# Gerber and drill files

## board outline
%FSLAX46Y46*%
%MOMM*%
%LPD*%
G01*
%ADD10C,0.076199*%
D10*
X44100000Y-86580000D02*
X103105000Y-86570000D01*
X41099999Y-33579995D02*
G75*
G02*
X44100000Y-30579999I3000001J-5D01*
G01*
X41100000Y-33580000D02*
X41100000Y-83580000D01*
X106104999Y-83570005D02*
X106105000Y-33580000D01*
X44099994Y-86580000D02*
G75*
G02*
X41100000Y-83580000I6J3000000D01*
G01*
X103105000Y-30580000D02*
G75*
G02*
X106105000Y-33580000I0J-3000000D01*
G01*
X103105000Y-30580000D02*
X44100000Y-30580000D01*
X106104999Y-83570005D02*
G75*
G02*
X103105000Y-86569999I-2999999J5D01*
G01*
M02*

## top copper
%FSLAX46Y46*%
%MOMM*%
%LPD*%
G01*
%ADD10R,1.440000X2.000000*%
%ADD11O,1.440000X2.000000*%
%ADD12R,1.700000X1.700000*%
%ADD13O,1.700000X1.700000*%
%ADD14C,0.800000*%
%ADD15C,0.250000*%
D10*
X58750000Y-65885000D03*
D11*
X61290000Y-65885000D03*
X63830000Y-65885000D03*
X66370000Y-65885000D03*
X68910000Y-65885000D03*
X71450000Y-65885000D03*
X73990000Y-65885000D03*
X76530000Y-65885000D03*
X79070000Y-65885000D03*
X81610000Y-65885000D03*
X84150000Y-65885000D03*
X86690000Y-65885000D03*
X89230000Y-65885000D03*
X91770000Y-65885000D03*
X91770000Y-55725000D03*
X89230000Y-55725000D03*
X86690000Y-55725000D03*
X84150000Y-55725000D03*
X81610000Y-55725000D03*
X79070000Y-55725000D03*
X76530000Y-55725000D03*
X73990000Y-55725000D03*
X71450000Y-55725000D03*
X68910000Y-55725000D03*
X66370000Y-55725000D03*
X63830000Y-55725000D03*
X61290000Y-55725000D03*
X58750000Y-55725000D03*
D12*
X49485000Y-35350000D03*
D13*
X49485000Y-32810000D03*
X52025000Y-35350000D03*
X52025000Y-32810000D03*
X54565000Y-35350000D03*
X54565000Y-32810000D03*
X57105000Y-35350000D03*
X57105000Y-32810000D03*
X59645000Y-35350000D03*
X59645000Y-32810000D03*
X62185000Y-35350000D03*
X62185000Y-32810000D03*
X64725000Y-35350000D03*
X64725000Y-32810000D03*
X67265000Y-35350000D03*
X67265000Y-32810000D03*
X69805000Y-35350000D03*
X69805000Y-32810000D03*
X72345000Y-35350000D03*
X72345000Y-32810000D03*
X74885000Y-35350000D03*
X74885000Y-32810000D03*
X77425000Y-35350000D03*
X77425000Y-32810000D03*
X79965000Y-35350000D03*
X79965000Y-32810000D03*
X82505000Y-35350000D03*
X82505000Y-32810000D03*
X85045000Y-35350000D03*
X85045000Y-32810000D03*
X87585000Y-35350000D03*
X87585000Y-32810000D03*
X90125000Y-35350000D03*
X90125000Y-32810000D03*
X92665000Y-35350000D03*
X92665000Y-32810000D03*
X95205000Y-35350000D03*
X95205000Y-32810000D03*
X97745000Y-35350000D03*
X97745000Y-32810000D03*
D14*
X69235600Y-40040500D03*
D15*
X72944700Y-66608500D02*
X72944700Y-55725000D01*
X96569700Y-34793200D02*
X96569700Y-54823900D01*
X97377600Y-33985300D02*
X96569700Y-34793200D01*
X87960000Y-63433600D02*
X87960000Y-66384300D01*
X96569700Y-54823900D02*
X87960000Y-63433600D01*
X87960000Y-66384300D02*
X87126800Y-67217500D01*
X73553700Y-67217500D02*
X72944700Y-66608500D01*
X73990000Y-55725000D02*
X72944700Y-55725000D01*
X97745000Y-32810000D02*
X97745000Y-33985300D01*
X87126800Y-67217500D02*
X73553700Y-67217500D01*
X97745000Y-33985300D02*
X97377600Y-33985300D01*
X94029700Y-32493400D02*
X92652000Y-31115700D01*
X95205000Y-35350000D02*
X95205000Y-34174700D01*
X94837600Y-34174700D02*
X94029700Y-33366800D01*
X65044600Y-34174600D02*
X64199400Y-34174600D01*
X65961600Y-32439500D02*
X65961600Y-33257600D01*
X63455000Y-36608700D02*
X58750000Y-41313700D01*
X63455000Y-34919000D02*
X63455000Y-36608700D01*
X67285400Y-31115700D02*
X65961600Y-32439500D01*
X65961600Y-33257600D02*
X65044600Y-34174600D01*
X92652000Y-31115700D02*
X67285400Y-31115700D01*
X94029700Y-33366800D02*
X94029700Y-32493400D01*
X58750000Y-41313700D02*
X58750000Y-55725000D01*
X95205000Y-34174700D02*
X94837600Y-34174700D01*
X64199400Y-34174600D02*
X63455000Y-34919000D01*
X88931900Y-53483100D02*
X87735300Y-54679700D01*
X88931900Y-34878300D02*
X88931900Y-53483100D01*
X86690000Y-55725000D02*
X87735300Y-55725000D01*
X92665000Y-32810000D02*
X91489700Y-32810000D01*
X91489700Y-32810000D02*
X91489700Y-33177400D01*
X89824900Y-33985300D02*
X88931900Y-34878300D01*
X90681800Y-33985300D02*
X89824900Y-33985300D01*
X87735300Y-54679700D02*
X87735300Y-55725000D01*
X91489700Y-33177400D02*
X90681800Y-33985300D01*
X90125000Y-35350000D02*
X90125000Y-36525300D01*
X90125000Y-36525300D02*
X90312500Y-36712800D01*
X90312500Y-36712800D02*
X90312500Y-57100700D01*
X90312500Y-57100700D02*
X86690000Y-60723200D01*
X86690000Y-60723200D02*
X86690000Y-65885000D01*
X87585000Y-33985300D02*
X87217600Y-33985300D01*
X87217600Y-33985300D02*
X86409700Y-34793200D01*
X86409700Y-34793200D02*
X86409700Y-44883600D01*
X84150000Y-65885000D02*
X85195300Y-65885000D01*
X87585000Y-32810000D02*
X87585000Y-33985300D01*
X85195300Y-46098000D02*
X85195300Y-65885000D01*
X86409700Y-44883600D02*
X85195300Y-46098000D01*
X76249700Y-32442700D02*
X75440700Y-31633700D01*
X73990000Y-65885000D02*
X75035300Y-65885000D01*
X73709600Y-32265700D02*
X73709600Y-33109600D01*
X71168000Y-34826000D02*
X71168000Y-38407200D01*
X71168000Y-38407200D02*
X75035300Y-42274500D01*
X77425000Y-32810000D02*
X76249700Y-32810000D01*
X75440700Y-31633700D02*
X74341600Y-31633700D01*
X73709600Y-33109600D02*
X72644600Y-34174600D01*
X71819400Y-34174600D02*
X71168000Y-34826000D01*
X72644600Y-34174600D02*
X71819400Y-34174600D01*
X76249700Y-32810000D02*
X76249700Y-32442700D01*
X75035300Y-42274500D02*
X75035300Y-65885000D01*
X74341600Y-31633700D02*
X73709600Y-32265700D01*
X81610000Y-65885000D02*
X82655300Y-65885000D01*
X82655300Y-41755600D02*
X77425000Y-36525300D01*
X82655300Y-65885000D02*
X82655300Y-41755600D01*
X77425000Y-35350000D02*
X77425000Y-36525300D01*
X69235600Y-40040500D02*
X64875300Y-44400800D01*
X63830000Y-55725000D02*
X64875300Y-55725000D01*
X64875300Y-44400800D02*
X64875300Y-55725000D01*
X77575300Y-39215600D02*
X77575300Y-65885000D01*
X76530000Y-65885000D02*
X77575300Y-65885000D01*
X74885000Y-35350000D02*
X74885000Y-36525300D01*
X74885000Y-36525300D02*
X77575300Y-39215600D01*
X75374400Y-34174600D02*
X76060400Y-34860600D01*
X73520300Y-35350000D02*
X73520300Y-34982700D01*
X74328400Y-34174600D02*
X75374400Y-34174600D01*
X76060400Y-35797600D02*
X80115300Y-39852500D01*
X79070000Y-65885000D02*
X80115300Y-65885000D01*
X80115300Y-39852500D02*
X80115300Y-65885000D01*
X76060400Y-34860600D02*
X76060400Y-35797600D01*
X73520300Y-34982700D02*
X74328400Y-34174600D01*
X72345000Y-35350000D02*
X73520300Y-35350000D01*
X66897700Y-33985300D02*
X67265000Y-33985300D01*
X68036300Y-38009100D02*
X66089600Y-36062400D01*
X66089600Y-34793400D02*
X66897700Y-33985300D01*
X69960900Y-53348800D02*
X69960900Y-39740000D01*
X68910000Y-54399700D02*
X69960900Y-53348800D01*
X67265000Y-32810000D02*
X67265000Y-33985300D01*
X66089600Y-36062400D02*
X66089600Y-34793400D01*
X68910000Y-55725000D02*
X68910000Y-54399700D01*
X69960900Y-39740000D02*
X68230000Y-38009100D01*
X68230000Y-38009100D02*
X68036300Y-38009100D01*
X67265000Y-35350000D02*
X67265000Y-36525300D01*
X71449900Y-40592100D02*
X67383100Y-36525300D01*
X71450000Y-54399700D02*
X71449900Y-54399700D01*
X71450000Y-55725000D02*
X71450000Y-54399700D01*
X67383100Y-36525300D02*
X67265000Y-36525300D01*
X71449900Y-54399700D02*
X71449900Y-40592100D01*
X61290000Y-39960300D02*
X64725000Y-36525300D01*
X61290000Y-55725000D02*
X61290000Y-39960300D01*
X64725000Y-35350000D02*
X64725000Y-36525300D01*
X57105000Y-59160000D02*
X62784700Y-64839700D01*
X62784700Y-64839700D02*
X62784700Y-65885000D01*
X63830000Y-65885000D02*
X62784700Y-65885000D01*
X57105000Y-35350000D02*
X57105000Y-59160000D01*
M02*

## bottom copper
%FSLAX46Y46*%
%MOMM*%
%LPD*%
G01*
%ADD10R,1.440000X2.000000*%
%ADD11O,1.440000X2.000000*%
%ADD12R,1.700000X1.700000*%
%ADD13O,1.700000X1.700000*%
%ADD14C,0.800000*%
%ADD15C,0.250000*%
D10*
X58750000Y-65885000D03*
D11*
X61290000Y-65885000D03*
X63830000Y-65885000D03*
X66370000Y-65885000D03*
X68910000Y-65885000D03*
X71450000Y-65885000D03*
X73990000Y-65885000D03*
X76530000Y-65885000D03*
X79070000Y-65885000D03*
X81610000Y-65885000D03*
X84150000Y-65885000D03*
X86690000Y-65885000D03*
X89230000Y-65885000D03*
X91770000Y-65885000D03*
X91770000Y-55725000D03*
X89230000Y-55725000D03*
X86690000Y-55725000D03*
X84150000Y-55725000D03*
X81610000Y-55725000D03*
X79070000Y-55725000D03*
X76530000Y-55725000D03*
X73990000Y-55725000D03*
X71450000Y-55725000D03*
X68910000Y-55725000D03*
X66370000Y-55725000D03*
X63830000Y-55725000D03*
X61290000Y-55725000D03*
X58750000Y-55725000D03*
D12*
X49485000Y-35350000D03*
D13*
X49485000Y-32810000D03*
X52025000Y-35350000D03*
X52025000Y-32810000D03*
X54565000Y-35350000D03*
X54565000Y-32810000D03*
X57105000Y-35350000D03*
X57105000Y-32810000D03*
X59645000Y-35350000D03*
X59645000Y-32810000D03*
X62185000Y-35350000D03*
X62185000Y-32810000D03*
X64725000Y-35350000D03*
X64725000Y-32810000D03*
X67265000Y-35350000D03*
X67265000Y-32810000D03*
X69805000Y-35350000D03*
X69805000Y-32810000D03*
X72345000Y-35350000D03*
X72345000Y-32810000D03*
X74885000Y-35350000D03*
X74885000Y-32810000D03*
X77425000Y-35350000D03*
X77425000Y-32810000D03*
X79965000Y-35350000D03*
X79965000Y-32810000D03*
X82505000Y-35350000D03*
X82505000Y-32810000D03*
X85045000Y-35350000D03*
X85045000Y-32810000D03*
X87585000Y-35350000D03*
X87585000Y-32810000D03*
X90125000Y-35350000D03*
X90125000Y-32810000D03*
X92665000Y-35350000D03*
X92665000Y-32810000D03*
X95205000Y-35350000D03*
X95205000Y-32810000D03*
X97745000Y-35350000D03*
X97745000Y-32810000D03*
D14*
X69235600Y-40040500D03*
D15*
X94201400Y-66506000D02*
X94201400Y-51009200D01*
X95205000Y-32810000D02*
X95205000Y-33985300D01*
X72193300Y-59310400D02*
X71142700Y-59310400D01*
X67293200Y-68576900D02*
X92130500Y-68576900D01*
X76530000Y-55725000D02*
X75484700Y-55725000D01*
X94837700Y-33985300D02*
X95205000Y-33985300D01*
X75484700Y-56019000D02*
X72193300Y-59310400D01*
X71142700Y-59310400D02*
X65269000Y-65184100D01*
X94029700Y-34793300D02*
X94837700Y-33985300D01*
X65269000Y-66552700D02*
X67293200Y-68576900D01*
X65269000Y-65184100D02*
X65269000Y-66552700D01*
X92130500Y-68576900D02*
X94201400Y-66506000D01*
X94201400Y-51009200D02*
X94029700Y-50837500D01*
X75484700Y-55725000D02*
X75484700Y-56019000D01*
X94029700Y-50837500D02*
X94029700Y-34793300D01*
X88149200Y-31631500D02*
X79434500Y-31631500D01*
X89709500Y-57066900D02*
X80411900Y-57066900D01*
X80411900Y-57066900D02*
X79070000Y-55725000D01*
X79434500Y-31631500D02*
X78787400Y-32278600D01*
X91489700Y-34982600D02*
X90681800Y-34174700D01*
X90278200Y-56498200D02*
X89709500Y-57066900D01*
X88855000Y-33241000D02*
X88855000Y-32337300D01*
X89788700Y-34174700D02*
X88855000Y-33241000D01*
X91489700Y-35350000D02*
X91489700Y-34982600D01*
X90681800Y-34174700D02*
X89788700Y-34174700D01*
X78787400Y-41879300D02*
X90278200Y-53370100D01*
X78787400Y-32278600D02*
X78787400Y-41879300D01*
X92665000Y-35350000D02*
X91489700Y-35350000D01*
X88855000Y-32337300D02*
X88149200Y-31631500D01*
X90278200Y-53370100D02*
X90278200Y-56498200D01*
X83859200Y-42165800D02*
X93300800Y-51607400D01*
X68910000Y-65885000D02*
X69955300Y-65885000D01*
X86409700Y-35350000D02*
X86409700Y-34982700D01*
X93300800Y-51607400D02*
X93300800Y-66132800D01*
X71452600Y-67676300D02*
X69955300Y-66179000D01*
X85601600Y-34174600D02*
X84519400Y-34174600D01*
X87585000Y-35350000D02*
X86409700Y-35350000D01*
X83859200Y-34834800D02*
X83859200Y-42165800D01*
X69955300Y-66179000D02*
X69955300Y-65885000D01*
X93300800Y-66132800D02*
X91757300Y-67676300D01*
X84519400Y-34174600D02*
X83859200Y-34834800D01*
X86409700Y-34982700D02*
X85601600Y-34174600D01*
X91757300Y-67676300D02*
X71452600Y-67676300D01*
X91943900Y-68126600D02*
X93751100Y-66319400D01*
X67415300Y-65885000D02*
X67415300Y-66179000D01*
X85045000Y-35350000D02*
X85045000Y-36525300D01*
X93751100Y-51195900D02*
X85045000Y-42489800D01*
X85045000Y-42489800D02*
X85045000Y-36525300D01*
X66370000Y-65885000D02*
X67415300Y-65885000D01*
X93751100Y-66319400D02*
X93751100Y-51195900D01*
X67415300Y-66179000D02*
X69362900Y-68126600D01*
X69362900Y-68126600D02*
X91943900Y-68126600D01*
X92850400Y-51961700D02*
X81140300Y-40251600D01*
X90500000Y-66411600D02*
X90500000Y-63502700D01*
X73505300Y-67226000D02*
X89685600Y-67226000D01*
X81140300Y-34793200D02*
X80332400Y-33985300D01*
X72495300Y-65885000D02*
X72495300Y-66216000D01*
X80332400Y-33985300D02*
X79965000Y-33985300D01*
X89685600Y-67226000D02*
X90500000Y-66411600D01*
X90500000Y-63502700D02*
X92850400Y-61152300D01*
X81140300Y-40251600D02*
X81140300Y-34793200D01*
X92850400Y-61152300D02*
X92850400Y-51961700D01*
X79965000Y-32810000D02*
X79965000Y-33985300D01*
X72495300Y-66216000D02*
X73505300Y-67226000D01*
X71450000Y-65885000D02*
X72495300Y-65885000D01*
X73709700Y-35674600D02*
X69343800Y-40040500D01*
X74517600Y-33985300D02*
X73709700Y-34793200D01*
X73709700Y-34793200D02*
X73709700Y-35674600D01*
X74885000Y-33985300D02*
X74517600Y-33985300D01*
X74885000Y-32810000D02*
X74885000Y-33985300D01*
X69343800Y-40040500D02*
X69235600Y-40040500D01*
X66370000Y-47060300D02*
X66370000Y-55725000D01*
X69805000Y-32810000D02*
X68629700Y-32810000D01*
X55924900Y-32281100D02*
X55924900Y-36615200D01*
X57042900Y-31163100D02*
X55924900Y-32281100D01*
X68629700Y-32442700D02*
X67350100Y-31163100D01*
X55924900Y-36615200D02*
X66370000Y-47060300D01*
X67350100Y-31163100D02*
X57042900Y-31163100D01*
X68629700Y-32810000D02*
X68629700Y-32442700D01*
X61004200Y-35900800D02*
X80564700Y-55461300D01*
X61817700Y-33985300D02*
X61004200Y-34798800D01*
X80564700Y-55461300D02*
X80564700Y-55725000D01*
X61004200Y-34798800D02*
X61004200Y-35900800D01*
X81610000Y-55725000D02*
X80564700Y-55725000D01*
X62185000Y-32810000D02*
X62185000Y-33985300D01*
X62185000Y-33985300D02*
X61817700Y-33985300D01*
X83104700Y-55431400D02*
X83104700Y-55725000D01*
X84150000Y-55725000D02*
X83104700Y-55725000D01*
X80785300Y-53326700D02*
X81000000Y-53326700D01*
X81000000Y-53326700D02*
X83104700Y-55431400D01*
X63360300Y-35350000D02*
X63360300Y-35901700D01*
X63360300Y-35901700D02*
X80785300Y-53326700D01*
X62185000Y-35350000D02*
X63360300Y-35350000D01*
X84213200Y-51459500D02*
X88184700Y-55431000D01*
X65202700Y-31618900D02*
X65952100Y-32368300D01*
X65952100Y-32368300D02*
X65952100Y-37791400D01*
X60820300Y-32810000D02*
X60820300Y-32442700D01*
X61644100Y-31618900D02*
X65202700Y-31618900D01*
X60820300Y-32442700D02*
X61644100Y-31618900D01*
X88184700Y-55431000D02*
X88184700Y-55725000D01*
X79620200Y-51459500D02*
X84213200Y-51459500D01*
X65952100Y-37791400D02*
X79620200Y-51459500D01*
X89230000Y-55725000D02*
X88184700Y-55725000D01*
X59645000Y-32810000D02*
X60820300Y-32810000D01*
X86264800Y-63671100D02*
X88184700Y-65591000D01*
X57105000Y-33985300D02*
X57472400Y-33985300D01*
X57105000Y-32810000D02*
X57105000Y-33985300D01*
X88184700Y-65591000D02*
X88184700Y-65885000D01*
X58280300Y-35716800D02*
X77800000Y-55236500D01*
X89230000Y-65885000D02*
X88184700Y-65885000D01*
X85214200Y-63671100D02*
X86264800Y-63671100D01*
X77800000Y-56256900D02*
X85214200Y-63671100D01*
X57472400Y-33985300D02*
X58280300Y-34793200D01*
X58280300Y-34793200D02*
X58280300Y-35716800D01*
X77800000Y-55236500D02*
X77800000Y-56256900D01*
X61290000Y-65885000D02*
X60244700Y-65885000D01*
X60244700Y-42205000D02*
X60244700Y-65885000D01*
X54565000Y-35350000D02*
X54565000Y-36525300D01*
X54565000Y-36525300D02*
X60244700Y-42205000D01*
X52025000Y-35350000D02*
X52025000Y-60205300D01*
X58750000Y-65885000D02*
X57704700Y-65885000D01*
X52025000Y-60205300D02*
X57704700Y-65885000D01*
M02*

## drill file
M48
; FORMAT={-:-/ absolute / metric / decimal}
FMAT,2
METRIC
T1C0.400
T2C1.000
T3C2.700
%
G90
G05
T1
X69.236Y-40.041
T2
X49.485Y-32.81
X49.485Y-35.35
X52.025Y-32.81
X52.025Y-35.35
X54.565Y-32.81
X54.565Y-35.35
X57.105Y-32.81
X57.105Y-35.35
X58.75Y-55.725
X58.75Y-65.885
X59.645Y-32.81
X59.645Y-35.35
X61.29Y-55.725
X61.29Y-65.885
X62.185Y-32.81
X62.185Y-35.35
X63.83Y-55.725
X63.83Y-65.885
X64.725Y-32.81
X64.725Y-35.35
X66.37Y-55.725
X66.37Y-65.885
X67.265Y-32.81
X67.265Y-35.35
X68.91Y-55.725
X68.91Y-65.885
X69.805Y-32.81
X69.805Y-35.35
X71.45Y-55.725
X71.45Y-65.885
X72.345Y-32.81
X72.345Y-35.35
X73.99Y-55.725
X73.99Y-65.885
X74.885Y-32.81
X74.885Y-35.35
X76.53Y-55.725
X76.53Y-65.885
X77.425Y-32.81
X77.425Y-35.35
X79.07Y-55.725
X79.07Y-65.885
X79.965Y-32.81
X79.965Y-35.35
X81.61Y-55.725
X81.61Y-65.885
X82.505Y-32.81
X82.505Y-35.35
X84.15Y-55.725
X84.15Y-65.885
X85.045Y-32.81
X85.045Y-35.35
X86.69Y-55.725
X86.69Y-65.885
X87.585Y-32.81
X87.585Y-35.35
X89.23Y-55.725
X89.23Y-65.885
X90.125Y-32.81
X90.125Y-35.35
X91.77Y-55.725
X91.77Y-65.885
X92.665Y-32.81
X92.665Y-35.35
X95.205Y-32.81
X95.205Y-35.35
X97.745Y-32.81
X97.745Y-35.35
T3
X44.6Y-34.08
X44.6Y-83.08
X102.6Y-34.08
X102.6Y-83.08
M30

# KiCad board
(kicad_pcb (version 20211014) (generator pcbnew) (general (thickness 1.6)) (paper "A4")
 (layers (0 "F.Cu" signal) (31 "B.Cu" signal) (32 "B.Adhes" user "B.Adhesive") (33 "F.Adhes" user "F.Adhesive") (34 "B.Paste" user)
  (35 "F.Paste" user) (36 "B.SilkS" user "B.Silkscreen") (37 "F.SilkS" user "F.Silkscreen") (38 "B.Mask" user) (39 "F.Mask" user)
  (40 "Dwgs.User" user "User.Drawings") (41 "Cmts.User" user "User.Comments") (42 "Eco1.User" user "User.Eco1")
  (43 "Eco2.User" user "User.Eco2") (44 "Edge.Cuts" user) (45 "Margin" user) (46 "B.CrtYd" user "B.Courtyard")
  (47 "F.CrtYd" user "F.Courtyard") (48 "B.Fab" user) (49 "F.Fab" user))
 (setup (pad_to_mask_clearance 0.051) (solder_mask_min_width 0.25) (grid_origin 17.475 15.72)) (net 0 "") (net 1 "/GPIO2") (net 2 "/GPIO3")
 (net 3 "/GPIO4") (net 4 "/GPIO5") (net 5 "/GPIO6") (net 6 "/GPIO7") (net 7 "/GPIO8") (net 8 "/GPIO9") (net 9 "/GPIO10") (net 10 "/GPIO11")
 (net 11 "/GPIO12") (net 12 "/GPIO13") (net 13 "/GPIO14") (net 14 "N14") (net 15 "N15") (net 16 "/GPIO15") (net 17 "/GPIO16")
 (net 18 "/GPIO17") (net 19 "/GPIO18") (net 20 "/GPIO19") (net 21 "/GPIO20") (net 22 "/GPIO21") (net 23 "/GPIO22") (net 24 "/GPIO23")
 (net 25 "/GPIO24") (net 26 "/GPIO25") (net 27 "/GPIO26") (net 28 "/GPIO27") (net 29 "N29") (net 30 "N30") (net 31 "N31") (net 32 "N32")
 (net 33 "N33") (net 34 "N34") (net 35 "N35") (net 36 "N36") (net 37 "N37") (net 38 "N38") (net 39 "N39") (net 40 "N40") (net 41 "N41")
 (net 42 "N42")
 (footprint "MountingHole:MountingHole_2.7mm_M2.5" (layer "F.Cu") (at 44.6 34.08)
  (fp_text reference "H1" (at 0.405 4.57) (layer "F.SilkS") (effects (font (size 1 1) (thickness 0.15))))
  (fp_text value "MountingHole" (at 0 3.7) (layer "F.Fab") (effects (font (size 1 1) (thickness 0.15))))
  (pad "" np_thru_hole circle locked (at 0 0) (size 2.7 2.7) (drill 2.7) (layers *.Cu *.Mask)))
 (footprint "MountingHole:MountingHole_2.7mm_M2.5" (layer "F.Cu") (at 44.6 83.08)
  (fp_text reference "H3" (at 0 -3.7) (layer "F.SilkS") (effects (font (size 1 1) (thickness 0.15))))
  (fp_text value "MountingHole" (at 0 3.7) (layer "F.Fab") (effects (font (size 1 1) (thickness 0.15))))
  (pad "" np_thru_hole circle locked (at 0 0) (size 2.7 2.7) (drill 2.7) (layers *.Cu *.Mask)))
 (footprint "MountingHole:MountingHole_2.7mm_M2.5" (layer "F.Cu") (at 102.6 34.08)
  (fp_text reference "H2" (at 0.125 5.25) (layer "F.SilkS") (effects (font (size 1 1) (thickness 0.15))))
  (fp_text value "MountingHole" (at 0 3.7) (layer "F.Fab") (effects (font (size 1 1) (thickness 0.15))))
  (pad "" np_thru_hole circle locked (at 0 0) (size 2.7 2.7) (drill 2.7) (layers *.Cu *.Mask)))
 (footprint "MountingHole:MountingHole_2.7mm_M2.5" (layer "F.Cu") (at 102.6 83.08)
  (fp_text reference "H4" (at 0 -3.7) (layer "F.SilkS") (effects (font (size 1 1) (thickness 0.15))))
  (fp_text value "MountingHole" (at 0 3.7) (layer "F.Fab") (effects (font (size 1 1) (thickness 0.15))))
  (pad "" np_thru_hole circle locked (at 0 0) (size 2.7 2.7) (drill 2.7) (layers *.Cu *.Mask)))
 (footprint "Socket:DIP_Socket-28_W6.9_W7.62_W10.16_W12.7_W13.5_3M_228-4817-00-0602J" (layer "F.Cu") (at 58.75 65.885 90)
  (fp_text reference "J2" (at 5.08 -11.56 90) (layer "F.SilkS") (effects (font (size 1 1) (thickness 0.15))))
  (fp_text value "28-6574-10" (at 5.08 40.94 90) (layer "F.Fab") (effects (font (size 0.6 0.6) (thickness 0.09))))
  (pad "1" thru_hole rect locked (at 0 0 90) (size 2 1.44) (drill 1) (layers *.Cu *.Mask) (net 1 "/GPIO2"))
  (pad "2" thru_hole oval locked (at 0 2.54 90) (size 2 1.44) (drill 1) (layers *.Cu *.Mask) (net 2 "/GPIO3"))
  (pad "3" thru_hole oval locked (at 0 5.08 90) (size 2 1.44) (drill 1) (layers *.Cu *.Mask) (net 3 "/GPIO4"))
  (pad "4" thru_hole oval locked (at 0 7.62 90) (size 2 1.44) (drill 1) (layers *.Cu *.Mask) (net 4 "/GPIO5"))
  (pad "5" thru_hole oval locked (at 0 10.16 90) (size 2 1.44) (drill 1) (layers *.Cu *.Mask) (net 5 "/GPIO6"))
  (pad "6" thru_hole oval locked (at 0 12.7 90) (size 2 1.44) (drill 1) (layers *.Cu *.Mask) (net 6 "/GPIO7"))
  (pad "7" thru_hole oval locked (at 0 15.24 90) (size 2 1.44) (drill 1) (layers *.Cu *.Mask) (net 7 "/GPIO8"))
  (pad "8" thru_hole oval locked (at 0 17.78 90) (size 2 1.44) (drill 1) (layers *.Cu *.Mask) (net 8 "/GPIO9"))
  (pad "9" thru_hole oval locked (at 0 20.32 90) (size 2 1.44) (drill 1) (layers *.Cu *.Mask) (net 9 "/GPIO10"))
  (pad "10" thru_hole oval locked (at 0 22.86 90) (size 2 1.44) (drill 1) (layers *.Cu *.Mask) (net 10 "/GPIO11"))
  (pad "11" thru_hole oval locked (at 0 25.4 90) (size 2 1.44) (drill 1) (layers *.Cu *.Mask) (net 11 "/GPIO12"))
  (pad "12" thru_hole oval locked (at 0 27.94 90) (size 2 1.44) (drill 1) (layers *.Cu *.Mask) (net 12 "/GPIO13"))
  (pad "13" thru_hole oval locked (at 0 30.48 90) (size 2 1.44) (drill 1) (layers *.Cu *.Mask) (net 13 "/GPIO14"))
  (pad "14" thru_hole oval locked (at 0 33.02 90) (size 2 1.44) (drill 1) (layers *.Cu *.Mask) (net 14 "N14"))
  (pad "15" thru_hole oval locked (at 10.16 33.02 90) (size 2 1.44) (drill 1) (layers *.Cu *.Mask) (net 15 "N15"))
  (pad "16" thru_hole oval locked (at 10.16 30.48 90) (size 2 1.44) (drill 1) (layers *.Cu *.Mask) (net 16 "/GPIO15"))
  (pad "17" thru_hole oval locked (at 10.16 27.94 90) (size 2 1.44) (drill 1) (layers *.Cu *.Mask) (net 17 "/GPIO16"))
  (pad "18" thru_hole oval locked (at 10.16 25.4 90) (size 2 1.44) (drill 1) (layers *.Cu *.Mask) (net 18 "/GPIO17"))
  (pad "19" thru_hole oval locked (at 10.16 22.86 90) (size 2 1.44) (drill 1) (layers *.Cu *.Mask) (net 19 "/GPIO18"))
  (pad "20" thru_hole oval locked (at 10.16 20.32 90) (size 2 1.44) (drill 1) (layers *.Cu *.Mask) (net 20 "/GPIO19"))
  (pad "21" thru_hole oval locked (at 10.16 17.78 90) (size 2 1.44) (drill 1) (layers *.Cu *.Mask) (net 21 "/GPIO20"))
  (pad "22" thru_hole oval locked (at 10.16 15.24 90) (size 2 1.44) (drill 1) (layers *.Cu *.Mask) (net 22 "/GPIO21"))
  (pad "23" thru_hole oval locked (at 10.16 12.7 90) (size 2 1.44) (drill 1) (layers *.Cu *.Mask) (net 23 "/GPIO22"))
  (pad "24" thru_hole oval locked (at 10.16 10.16 90) (size 2 1.44) (drill 1) (layers *.Cu *.Mask) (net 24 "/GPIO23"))
  (pad "25" thru_hole oval locked (at 10.16 7.62 90) (size 2 1.44) (drill 1) (layers *.Cu *.Mask) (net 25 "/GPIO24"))
  (pad "26" thru_hole oval locked (at 10.16 5.08 90) (size 2 1.44) (drill 1) (layers *.Cu *.Mask) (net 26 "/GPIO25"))
  (pad "27" thru_hole oval locked (at 10.16 2.54 90) (size 2 1.44) (drill 1) (layers *.Cu *.Mask) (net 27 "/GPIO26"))
  (pad "28" thru_hole oval locked (at 10.16 0 90) (size 2 1.44) (drill 1) (layers *.Cu *.Mask) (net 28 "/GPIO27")))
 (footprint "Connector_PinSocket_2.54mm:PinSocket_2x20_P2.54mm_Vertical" (layer "B.Cu") (at 49.485 35.35 -90)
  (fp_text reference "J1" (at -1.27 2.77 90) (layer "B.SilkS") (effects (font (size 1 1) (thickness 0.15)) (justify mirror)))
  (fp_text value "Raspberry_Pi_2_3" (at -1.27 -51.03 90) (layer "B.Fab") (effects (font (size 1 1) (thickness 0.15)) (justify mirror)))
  (pad "1" thru_hole rect locked (at 0 0 270) (size 1.7 1.7) (drill 1) (layers *.Cu *.Mask) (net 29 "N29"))
  (pad "2" thru_hole oval locked (at -2.54 0 270) (size 1.7 1.7) (drill 1) (layers *.Cu *.Mask) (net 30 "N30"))
  (pad "3" thru_hole oval locked (at 0 -2.54 270) (size 1.7 1.7) (drill 1) (layers *.Cu *.Mask) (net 1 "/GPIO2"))
  (pad "4" thru_hole oval locked (at -2.54 -2.54 270) (size 1.7 1.7) (drill 1) (layers *.Cu *.Mask) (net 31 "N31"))
  (pad "5" thru_hole oval locked (at 0 -5.08 270) (size 1.7 1.7) (drill 1) (layers *.Cu *.Mask) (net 2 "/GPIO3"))
  (pad "6" thru_hole oval locked (at -2.54 -5.08 270) (size 1.7 1.7) (drill 1) (layers *.Cu *.Mask) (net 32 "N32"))
  (pad "7" thru_hole oval locked (at 0 -7.62 270) (size 1.7 1.7) (drill 1) (layers *.Cu *.Mask) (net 3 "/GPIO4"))
  (pad "8" thru_hole oval locked (at -2.54 -7.62 270) (size 1.7 1.7) (drill 1) (layers *.Cu *.Mask) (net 13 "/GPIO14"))
  (pad "9" thru_hole oval locked (at 0 -10.16 270) (size 1.7 1.7) (drill 1) (layers *.Cu *.Mask) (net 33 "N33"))
  (pad "10" thru_hole oval locked (at -2.54 -10.16 270) (size 1.7 1.7) (drill 1) (layers *.Cu *.Mask) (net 16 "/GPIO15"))
  (pad "11" thru_hole oval locked (at 0 -12.7 270) (size 1.7 1.7) (drill 1) (layers *.Cu *.Mask) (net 18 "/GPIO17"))
  (pad "12" thru_hole oval locked (at -2.54 -12.7 270) (size 1.7 1.7) (drill 1) (layers *.Cu *.Mask) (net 19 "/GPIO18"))
  (pad "13" thru_hole oval locked (at 0 -15.24 270) (size 1.7 1.7) (drill 1) (layers *.Cu *.Mask) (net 27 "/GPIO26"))
  (pad "14" thru_hole oval locked (at -2.54 -15.24 270) (size 1.7 1.7) (drill 1) (layers *.Cu *.Mask) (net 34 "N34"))
  (pad "15" thru_hole oval locked (at 0 -17.78 270) (size 1.7 1.7) (drill 1) (layers *.Cu *.Mask) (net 23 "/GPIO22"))
  (pad "16" thru_hole oval locked (at -2.54 -17.78 270) (size 1.7 1.7) (drill 1) (layers *.Cu *.Mask) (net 24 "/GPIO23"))
  (pad "17" thru_hole oval locked (at 0 -20.32 270) (size 1.7 1.7) (drill 1) (layers *.Cu *.Mask) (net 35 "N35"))
  (pad "18" thru_hole oval locked (at -2.54 -20.32 270) (size 1.7 1.7) (drill 1) (layers *.Cu *.Mask) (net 25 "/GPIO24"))
  (pad "19" thru_hole oval locked (at 0 -22.86 270) (size 1.7 1.7) (drill 1) (layers *.Cu *.Mask) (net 9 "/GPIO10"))
  (pad "20" thru_hole oval locked (at -2.54 -22.86 270) (size 1.7 1.7) (drill 1) (layers *.Cu *.Mask) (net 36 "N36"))
  (pad "21" thru_hole oval locked (at 0 -25.4 270) (size 1.7 1.7) (drill 1) (layers *.Cu *.Mask) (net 8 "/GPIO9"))
  (pad "22" thru_hole oval locked (at -2.54 -25.4 270) (size 1.7 1.7) (drill 1) (layers *.Cu *.Mask) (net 26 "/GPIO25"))
  (pad "23" thru_hole oval locked (at 0 -27.94 270) (size 1.7 1.7) (drill 1) (layers *.Cu *.Mask) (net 10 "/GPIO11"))
  (pad "24" thru_hole oval locked (at -2.54 -27.94 270) (size 1.7 1.7) (drill 1) (layers *.Cu *.Mask) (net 7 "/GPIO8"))
  (pad "25" thru_hole oval locked (at 0 -30.48 270) (size 1.7 1.7) (drill 1) (layers *.Cu *.Mask) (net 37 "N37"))
  (pad "26" thru_hole oval locked (at -2.54 -30.48 270) (size 1.7 1.7) (drill 1) (layers *.Cu *.Mask) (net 6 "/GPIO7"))
  (pad "27" thru_hole oval locked (at 0 -33.02 270) (size 1.7 1.7) (drill 1) (layers *.Cu *.Mask) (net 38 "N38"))
  (pad "28" thru_hole oval locked (at -2.54 -33.02 270) (size 1.7 1.7) (drill 1) (layers *.Cu *.Mask) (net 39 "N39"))
  (pad "29" thru_hole oval locked (at 0 -35.56 270) (size 1.7 1.7) (drill 1) (layers *.Cu *.Mask) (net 4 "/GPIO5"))
  (pad "30" thru_hole oval locked (at -2.54 -35.56 270) (size 1.7 1.7) (drill 1) (layers *.Cu *.Mask) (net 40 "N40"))
  (pad "31" thru_hole oval locked (at 0 -38.1 270) (size 1.7 1.7) (drill 1) (layers *.Cu *.Mask) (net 5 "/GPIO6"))
  (pad "32" thru_hole oval locked (at -2.54 -38.1 270) (size 1.7 1.7) (drill 1) (layers *.Cu *.Mask) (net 11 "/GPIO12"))
  (pad "33" thru_hole oval locked (at 0 -40.64 270) (size 1.7 1.7) (drill 1) (layers *.Cu *.Mask) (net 12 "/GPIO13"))
  (pad "34" thru_hole oval locked (at -2.54 -40.64 270) (size 1.7 1.7) (drill 1) (layers *.Cu *.Mask) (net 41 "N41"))
  (pad "35" thru_hole oval locked (at 0 -43.18 270) (size 1.7 1.7) (drill 1) (layers *.Cu *.Mask) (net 20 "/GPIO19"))
  (pad "36" thru_hole oval locked (at -2.54 -43.18 270) (size 1.7 1.7) (drill 1) (layers *.Cu *.Mask) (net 17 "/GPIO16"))
  (pad "37" thru_hole oval locked (at 0 -45.72 270) (size 1.7 1.7) (drill 1) (layers *.Cu *.Mask) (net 28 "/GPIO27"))
  (pad "38" thru_hole oval locked (at -2.54 -45.72 270) (size 1.7 1.7) (drill 1) (layers *.Cu *.Mask) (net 21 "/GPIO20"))
  (pad "39" thru_hole oval locked (at 0 -48.26 270) (size 1.7 1.7) (drill 1) (layers *.Cu *.Mask) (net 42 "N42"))
  (pad "40" thru_hole oval locked (at -2.54 -48.26 270) (size 1.7 1.7) (drill 1) (layers *.Cu *.Mask) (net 22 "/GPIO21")))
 (gr_line (start 44.1 86.58) (end 103.105 86.57) (layer "Edge.Cuts") (width 0.076199))
 (gr_arc (start 41.099999 33.579995) (mid 41.97868 31.458677) (end 44.1 30.58) (layer "Edge.Cuts") (width 0.076199))
 (gr_line (start 41.1 33.58) (end 41.1 83.58) (layer "Edge.Cuts") (width 0.076199))
 (gr_line (start 106.104999 83.570005) (end 106.105 33.58) (layer "Edge.Cuts") (width 0.076199))
 (gr_arc (start 44.099994 86.58) (mid 41.978677 85.701319) (end 41.1 83.58) (layer "Edge.Cuts") (width 0.076199))
 (gr_arc (start 103.105 30.58) (mid 105.226318 31.45868) (end 106.104996 33.58) (layer "Edge.Cuts") (width 0.076199))
 (gr_line (start 103.105 30.58) (end 44.1 30.58) (layer "Edge.Cuts") (width 0.076199))
 (gr_arc (start 106.104999 83.570005) (mid 105.226319 85.691323) (end 103.105 86.57) (layer "Edge.Cuts") (width 0.076199))
 (segment (start 72.9447 66.6085) (end 72.9447 55.725) (width 0.25) (layer "F.Cu") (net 22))
 (segment (start 96.5697 34.7932) (end 96.5697 54.8239) (width 0.25) (layer "F.Cu") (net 22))
 (segment (start 97.3776 33.9853) (end 96.5697 34.7932) (width 0.25) (layer "F.Cu") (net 22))
 (segment (start 87.96 63.4336) (end 87.96 66.3843) (width 0.25) (layer "F.Cu") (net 22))
 (segment (start 96.5697 54.8239) (end 87.96 63.4336) (width 0.25) (layer "F.Cu") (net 22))
 (segment (start 87.96 66.3843) (end 87.1268 67.2175) (width 0.25) (layer "F.Cu") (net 22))
 (segment (start 73.5537 67.2175) (end 72.9447 66.6085) (width 0.25) (layer "F.Cu") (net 22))
 (segment (start 73.99 55.725) (end 72.9447 55.725) (width 0.25) (layer "F.Cu") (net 22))
 (segment (start 97.745 32.81) (end 97.745 33.9853) (width 0.25) (layer "F.Cu") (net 22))
 (segment (start 87.1268 67.2175) (end 73.5537 67.2175) (width 0.25) (layer "F.Cu") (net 22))
 (segment (start 97.745 33.9853) (end 97.3776 33.9853) (width 0.25) (layer "F.Cu") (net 22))
 (segment (start 94.2014 66.506) (end 94.2014 51.0092) (width 0.25) (layer "B.Cu") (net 21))
 (segment (start 95.205 32.81) (end 95.205 33.9853) (width 0.25) (layer "B.Cu") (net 21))
 (segment (start 72.1933 59.3104) (end 71.1427 59.3104) (width 0.25) (layer "B.Cu") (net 21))
 (segment (start 67.2932 68.5769) (end 92.1305 68.5769) (width 0.25) (layer "B.Cu") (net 21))
 (segment (start 76.53 55.725) (end 75.4847 55.725) (width 0.25) (layer "B.Cu") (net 21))
 (segment (start 94.8377 33.9853) (end 95.205 33.9853) (width 0.25) (layer "B.Cu") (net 21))
 (segment (start 75.4847 56.019) (end 72.1933 59.3104) (width 0.25) (layer "B.Cu") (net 21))
 (segment (start 71.1427 59.3104) (end 65.269 65.1841) (width 0.25) (layer "B.Cu") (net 21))
 (segment (start 94.0297 34.7933) (end 94.8377 33.9853) (width 0.25) (layer "B.Cu") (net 21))
 (segment (start 65.269 66.5527) (end 67.2932 68.5769) (width 0.25) (layer "B.Cu") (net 21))
 (segment (start 65.269 65.1841) (end 65.269 66.5527) (width 0.25) (layer "B.Cu") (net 21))
 (segment (start 92.1305 68.5769) (end 94.2014 66.506) (width 0.25) (layer "B.Cu") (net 21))
 (segment (start 94.2014 51.0092) (end 94.0297 50.8375) (width 0.25) (layer "B.Cu") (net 21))
 (segment (start 75.4847 55.725) (end 75.4847 56.019) (width 0.25) (layer "B.Cu") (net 21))
 (segment (start 94.0297 50.8375) (end 94.0297 34.7933) (width 0.25) (layer "B.Cu") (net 21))
 (segment (start 94.0297 32.4934) (end 92.652 31.1157) (width 0.25) (layer "F.Cu") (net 28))
 (segment (start 95.205 35.35) (end 95.205 34.1747) (width 0.25) (layer "F.Cu") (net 28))
 (segment (start 94.8376 34.1747) (end 94.0297 33.3668) (width 0.25) (layer "F.Cu") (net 28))
 (segment (start 65.0446 34.1746) (end 64.1994 34.1746) (width 0.25) (layer "F.Cu") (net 28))
 (segment (start 65.9616 32.4395) (end 65.9616 33.2576) (width 0.25) (layer "F.Cu") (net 28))
 (segment (start 63.455 36.6087) (end 58.75 41.3137) (width 0.25) (layer "F.Cu") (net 28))
 (segment (start 63.455 34.919) (end 63.455 36.6087) (width 0.25) (layer "F.Cu") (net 28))
 (segment (start 67.2854 31.1157) (end 65.9616 32.4395) (width 0.25) (layer "F.Cu") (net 28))
 (segment (start 65.9616 33.2576) (end 65.0446 34.1746) (width 0.25) (layer "F.Cu") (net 28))
 (segment (start 92.652 31.1157) (end 67.2854 31.1157) (width 0.25) (layer "F.Cu") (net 28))
 (segment (start 94.0297 33.3668) (end 94.0297 32.4934) (width 0.25) (layer "F.Cu") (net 28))
 (segment (start 58.75 41.3137) (end 58.75 55.725) (width 0.25) (layer "F.Cu") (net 28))
 (segment (start 95.205 34.1747) (end 94.8376 34.1747) (width 0.25) (layer "F.Cu") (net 28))
 (segment (start 64.1994 34.1746) (end 63.455 34.919) (width 0.25) (layer "F.Cu") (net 28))
 (segment (start 88.9319 53.4831) (end 87.7353 54.6797) (width 0.25) (layer "F.Cu") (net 17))
 (segment (start 88.9319 34.8783) (end 88.9319 53.4831) (width 0.25) (layer "F.Cu") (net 17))
 (segment (start 86.69 55.725) (end 87.7353 55.725) (width 0.25) (layer "F.Cu") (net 17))
 (segment (start 92.665 32.81) (end 91.4897 32.81) (width 0.25) (layer "F.Cu") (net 17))
 (segment (start 91.4897 32.81) (end 91.4897 33.1774) (width 0.25) (layer "F.Cu") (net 17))
 (segment (start 89.8249 33.9853) (end 88.9319 34.8783) (width 0.25) (layer "F.Cu") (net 17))
 (segment (start 90.6818 33.9853) (end 89.8249 33.9853) (width 0.25) (layer "F.Cu") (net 17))
 (segment (start 87.7353 54.6797) (end 87.7353 55.725) (width 0.25) (layer "F.Cu") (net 17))
 (segment (start 91.4897 33.1774) (end 90.6818 33.9853) (width 0.25) (layer "F.Cu") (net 17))
 (segment (start 88.1492 31.6315) (end 79.4345 31.6315) (width 0.25) (layer "B.Cu") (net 20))
 (segment (start 89.7095 57.0669) (end 80.4119 57.0669) (width 0.25) (layer "B.Cu") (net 20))
 (segment (start 80.4119 57.0669) (end 79.07 55.725) (width 0.25) (layer "B.Cu") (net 20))
 (segment (start 79.4345 31.6315) (end 78.7874 32.2786) (width 0.25) (layer "B.Cu") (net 20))
 (segment (start 91.4897 34.9826) (end 90.6818 34.1747) (width 0.25) (layer "B.Cu") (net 20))
 (segment (start 90.2782 56.4982) (end 89.7095 57.0669) (width 0.25) (layer "B.Cu") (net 20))
 (segment (start 88.855 33.241) (end 88.855 32.3373) (width 0.25) (layer "B.Cu") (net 20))
 (segment (start 89.7887 34.1747) (end 88.855 33.241) (width 0.25) (layer "B.Cu") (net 20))
 (segment (start 91.4897 35.35) (end 91.4897 34.9826) (width 0.25) (layer "B.Cu") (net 20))
 (segment (start 90.6818 34.1747) (end 89.7887 34.1747) (width 0.25) (layer "B.Cu") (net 20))
 (segment (start 78.7874 41.8793) (end 90.2782 53.3701) (width 0.25) (layer "B.Cu") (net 20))
 (segment (start 78.7874 32.2786) (end 78.7874 41.8793) (width 0.25) (layer "B.Cu") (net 20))
 (segment (start 92.665 35.35) (end 91.4897 35.35) (width 0.25) (layer "B.Cu") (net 20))
 (segment (start 88.855 32.3373) (end 88.1492 31.6315) (width 0.25) (layer "B.Cu") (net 20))
 (segment (start 90.2782 53.3701) (end 90.2782 56.4982) (width 0.25) (layer "B.Cu") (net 20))
 (segment (start 90.125 35.35) (end 90.125 36.5253) (width 0.25) (layer "F.Cu") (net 12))
 (segment (start 90.125 36.5253) (end 90.3125 36.7128) (width 0.25) (layer "F.Cu") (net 12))
 (segment (start 90.3125 36.7128) (end 90.3125 57.1007) (width 0.25) (layer "F.Cu") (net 12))
 (segment (start 90.3125 57.1007) (end 86.69 60.7232) (width 0.25) (layer "F.Cu") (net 12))
 (segment (start 86.69 60.7232) (end 86.69 65.885) (width 0.25) (layer "F.Cu") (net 12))
 (segment (start 87.585 33.9853) (end 87.2176 33.9853) (width 0.25) (layer "F.Cu") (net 11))
 (segment (start 87.2176 33.9853) (end 86.4097 34.7932) (width 0.25) (layer "F.Cu") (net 11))
 (segment (start 86.4097 34.7932) (end 86.4097 44.8836) (width 0.25) (layer "F.Cu") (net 11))
 (segment (start 84.15 65.885) (end 85.1953 65.885) (width 0.25) (layer "F.Cu") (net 11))
 (segment (start 87.585 32.81) (end 87.585 33.9853) (width 0.25) (layer "F.Cu") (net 11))
 (segment (start 85.1953 46.098) (end 85.1953 65.885) (width 0.25) (layer "F.Cu") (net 11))
 (segment (start 86.4097 44.8836) (end 85.1953 46.098) (width 0.25) (layer "F.Cu") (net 11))
 (segment (start 83.8592 42.1658) (end 93.3008 51.6074) (width 0.25) (layer "B.Cu") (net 5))
 (segment (start 68.91 65.885) (end 69.9553 65.885) (width 0.25) (layer "B.Cu") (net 5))
 (segment (start 86.4097 35.35) (end 86.4097 34.9827) (width 0.25) (layer "B.Cu") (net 5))
 (segment (start 93.3008 51.6074) (end 93.3008 66.1328) (width 0.25) (layer "B.Cu") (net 5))
 (segment (start 71.4526 67.6763) (end 69.9553 66.179) (width 0.25) (layer "B.Cu") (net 5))
 (segment (start 85.6016 34.1746) (end 84.5194 34.1746) (width 0.25) (layer "B.Cu") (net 5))
 (segment (start 87.585 35.35) (end 86.4097 35.35) (width 0.25) (layer "B.Cu") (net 5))
 (segment (start 83.8592 34.8348) (end 83.8592 42.1658) (width 0.25) (layer "B.Cu") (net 5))
 (segment (start 69.9553 66.179) (end 69.9553 65.885) (width 0.25) (layer "B.Cu") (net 5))
 (segment (start 93.3008 66.1328) (end 91.7573 67.6763) (width 0.25) (layer "B.Cu") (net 5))
 (segment (start 84.5194 34.1746) (end 83.8592 34.8348) (width 0.25) (layer "B.Cu") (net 5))
 (segment (start 86.4097 34.9827) (end 85.6016 34.1746) (width 0.25) (layer "B.Cu") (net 5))
 (segment (start 91.7573 67.6763) (end 71.4526 67.6763) (width 0.25) (layer "B.Cu") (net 5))
 (segment (start 91.9439 68.1266) (end 93.7511 66.3194) (width 0.25) (layer "B.Cu") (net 4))
 (segment (start 67.4153 65.885) (end 67.4153 66.179) (width 0.25) (layer "B.Cu") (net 4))
 (segment (start 85.045 35.35) (end 85.045 36.5253) (width 0.25) (layer "B.Cu") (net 4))
 (segment (start 93.7511 51.1959) (end 85.045 42.4898) (width 0.25) (layer "B.Cu") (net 4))
 (segment (start 85.045 42.4898) (end 85.045 36.5253) (width 0.25) (layer "B.Cu") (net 4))
 (segment (start 66.37 65.885) (end 67.4153 65.885) (width 0.25) (layer "B.Cu") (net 4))
 (segment (start 93.7511 66.3194) (end 93.7511 51.1959) (width 0.25) (layer "B.Cu") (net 4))
 (segment (start 67.4153 66.179) (end 69.3629 68.1266) (width 0.25) (layer "B.Cu") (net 4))
 (segment (start 69.3629 68.1266) (end 91.9439 68.1266) (width 0.25) (layer "B.Cu") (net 4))
 (segment (start 92.8504 51.9617) (end 81.1403 40.2516) (width 0.25) (layer "B.Cu") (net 6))
 (segment (start 90.5 66.4116) (end 90.5 63.5027) (width 0.25) (layer "B.Cu") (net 6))
 (segment (start 73.5053 67.226) (end 89.6856 67.226) (width 0.25) (layer "B.Cu") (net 6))
 (segment (start 81.1403 34.7932) (end 80.3324 33.9853) (width 0.25) (layer "B.Cu") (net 6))
 (segment (start 72.4953 65.885) (end 72.4953 66.216) (width 0.25) (layer "B.Cu") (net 6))
 (segment (start 80.3324 33.9853) (end 79.965 33.9853) (width 0.25) (layer "B.Cu") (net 6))
 (segment (start 89.6856 67.226) (end 90.5 66.4116) (width 0.25) (layer "B.Cu") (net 6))
 (segment (start 90.5 63.5027) (end 92.8504 61.1523) (width 0.25) (layer "B.Cu") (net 6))
 (segment (start 81.1403 40.2516) (end 81.1403 34.7932) (width 0.25) (layer "B.Cu") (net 6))
 (segment (start 92.8504 61.1523) (end 92.8504 51.9617) (width 0.25) (layer "B.Cu") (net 6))
 (segment (start 79.965 32.81) (end 79.965 33.9853) (width 0.25) (layer "B.Cu") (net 6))
 (segment (start 72.4953 66.216) (end 73.5053 67.226) (width 0.25) (layer "B.Cu") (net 6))
 (segment (start 71.45 65.885) (end 72.4953 65.885) (width 0.25) (layer "B.Cu") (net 6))
 (segment (start 76.2497 32.4427) (end 75.4407 31.6337) (width 0.25) (layer "F.Cu") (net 7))
 (segment (start 73.99 65.885) (end 75.0353 65.885) (width 0.25) (layer "F.Cu") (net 7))
 (segment (start 73.7096 32.2657) (end 73.7096 33.1096) (width 0.25) (layer "F.Cu") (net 7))
 (segment (start 71.168 34.826) (end 71.168 38.4072) (width 0.25) (layer "F.Cu") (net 7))
 (segment (start 71.168 38.4072) (end 75.0353 42.2745) (width 0.25) (layer "F.Cu") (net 7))
 (segment (start 77.425 32.81) (end 76.2497 32.81) (width 0.25) (layer "F.Cu") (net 7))
 (segment (start 75.4407 31.6337) (end 74.3416 31.6337) (width 0.25) (layer "F.Cu") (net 7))
 (segment (start 73.7096 33.1096) (end 72.6446 34.1746) (width 0.25) (layer "F.Cu") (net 7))
 (segment (start 71.8194 34.1746) (end 71.168 34.826) (width 0.25) (layer "F.Cu") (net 7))
 (segment (start 72.6446 34.1746) (end 71.8194 34.1746) (width 0.25) (layer "F.Cu") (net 7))
 (segment (start 76.2497 32.81) (end 76.2497 32.4427) (width 0.25) (layer "F.Cu") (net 7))
 (segment (start 75.0353 42.2745) (end 75.0353 65.885) (width 0.25) (layer "F.Cu") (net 7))
 (segment (start 74.3416 31.6337) (end 73.7096 32.2657) (width 0.25) (layer "F.Cu") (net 7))
 (segment (start 81.61 65.885) (end 82.6553 65.885) (width 0.25) (layer "F.Cu") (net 10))
 (segment (start 82.6553 41.7556) (end 77.425 36.5253) (width 0.25) (layer "F.Cu") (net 10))
 (segment (start 82.6553 65.885) (end 82.6553 41.7556) (width 0.25) (layer "F.Cu") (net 10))
 (segment (start 77.425 35.35) (end 77.425 36.5253) (width 0.25) (layer "F.Cu") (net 10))
 (segment (start 69.2356 40.0405) (end 64.8753 44.4008) (width 0.25) (layer "F.Cu") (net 26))
 (segment (start 63.83 55.725) (end 64.8753 55.725) (width 0.25) (layer "F.Cu") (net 26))
 (segment (start 64.8753 44.4008) (end 64.8753 55.725) (width 0.25) (layer "F.Cu") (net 26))
 (via (at 69.2356 40.0405) (size 0.8) (drill 0.4) (layers "F.Cu" "B.Cu") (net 26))
 (segment (start 73.7097 35.6746) (end 69.3438 40.0405) (width 0.25) (layer "B.Cu") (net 26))
 (segment (start 74.5176 33.9853) (end 73.7097 34.7932) (width 0.25) (layer "B.Cu") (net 26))
 (segment (start 73.7097 34.7932) (end 73.7097 35.6746) (width 0.25) (layer "B.Cu") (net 26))
 (segment (start 74.885 33.9853) (end 74.5176 33.9853) (width 0.25) (layer "B.Cu") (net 26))
 (segment (start 74.885 32.81) (end 74.885 33.9853) (width 0.25) (layer "B.Cu") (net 26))
 (segment (start 69.3438 40.0405) (end 69.2356 40.0405) (width 0.25) (layer "B.Cu") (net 26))
 (segment (start 77.5753 39.2156) (end 77.5753 65.885) (width 0.25) (layer "F.Cu") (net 8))
 (segment (start 76.53 65.885) (end 77.5753 65.885) (width 0.25) (layer "F.Cu") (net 8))
 (segment (start 74.885 35.35) (end 74.885 36.5253) (width 0.25) (layer "F.Cu") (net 8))
 (segment (start 74.885 36.5253) (end 77.5753 39.2156) (width 0.25) (layer "F.Cu") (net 8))
 (segment (start 75.3744 34.1746) (end 76.0604 34.8606) (width 0.25) (layer "F.Cu") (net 9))
 (segment (start 73.5203 35.35) (end 73.5203 34.9827) (width 0.25) (layer "F.Cu") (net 9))
 (segment (start 74.3284 34.1746) (end 75.3744 34.1746) (width 0.25) (layer "F.Cu") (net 9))
 (segment (start 76.0604 35.7976) (end 80.1153 39.8525) (width 0.25) (layer "F.Cu") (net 9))
 (segment (start 79.07 65.885) (end 80.1153 65.885) (width 0.25) (layer "F.Cu") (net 9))
 (segment (start 80.1153 39.8525) (end 80.1153 65.885) (width 0.25) (layer "F.Cu") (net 9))
 (segment (start 76.0604 34.8606) (end 76.0604 35.7976) (width 0.25) (layer "F.Cu") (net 9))
 (segment (start 73.5203 34.9827) (end 74.3284 34.1746) (width 0.25) (layer "F.Cu") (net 9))
 (segment (start 72.345 35.35) (end 73.5203 35.35) (width 0.25) (layer "F.Cu") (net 9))
 (segment (start 66.37 47.0603) (end 66.37 55.725) (width 0.25) (layer "B.Cu") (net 25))
 (segment (start 69.805 32.81) (end 68.6297 32.81) (width 0.25) (layer "B.Cu") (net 25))
 (segment (start 55.9249 32.2811) (end 55.9249 36.6152) (width 0.25) (layer "B.Cu") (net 25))
 (segment (start 57.0429 31.1631) (end 55.9249 32.2811) (width 0.25) (layer "B.Cu") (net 25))
 (segment (start 68.6297 32.4427) (end 67.3501 31.1631) (width 0.25) (layer "B.Cu") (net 25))
 (segment (start 55.9249 36.6152) (end 66.37 47.0603) (width 0.25) (layer "B.Cu") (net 25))
 (segment (start 67.3501 31.1631) (end 57.0429 31.1631) (width 0.25) (layer "B.Cu") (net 25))
 (segment (start 68.6297 32.81) (end 68.6297 32.4427) (width 0.25) (layer "B.Cu") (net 25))
 (segment (start 66.8977 33.9853) (end 67.265 33.9853) (width 0.25) (layer "F.Cu") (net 24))
 (segment (start 68.0363 38.0091) (end 66.0896 36.0624) (width 0.25) (layer "F.Cu") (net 24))
 (segment (start 66.0896 34.7934) (end 66.8977 33.9853) (width 0.25) (layer "F.Cu") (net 24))
 (segment (start 69.9609 53.3488) (end 69.9609 39.74) (width 0.25) (layer "F.Cu") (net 24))
 (segment (start 68.91 54.3997) (end 69.9609 53.3488) (width 0.25) (layer "F.Cu") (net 24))
 (segment (start 67.265 32.81) (end 67.265 33.9853) (width 0.25) (layer "F.Cu") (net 24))
 (segment (start 66.0896 36.0624) (end 66.0896 34.7934) (width 0.25) (layer "F.Cu") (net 24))
 (segment (start 68.91 55.725) (end 68.91 54.3997) (width 0.25) (layer "F.Cu") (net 24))
 (segment (start 69.9609 39.74) (end 68.23 38.0091) (width 0.25) (layer "F.Cu") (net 24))
 (segment (start 68.23 38.0091) (end 68.0363 38.0091) (width 0.25) (layer "F.Cu") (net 24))
 (segment (start 67.265 35.35) (end 67.265 36.5253) (width 0.25) (layer "F.Cu") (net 23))
 (segment (start 71.4499 40.5921) (end 67.3831 36.5253) (width 0.25) (layer "F.Cu") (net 23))
 (segment (start 71.45 54.3997) (end 71.4499 54.3997) (width 0.25) (layer "F.Cu") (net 23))
 (segment (start 71.45 55.725) (end 71.45 54.3997) (width 0.25) (layer "F.Cu") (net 23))
 (segment (start 67.3831 36.5253) (end 67.265 36.5253) (width 0.25) (layer "F.Cu") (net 23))
 (segment (start 71.4499 54.3997) (end 71.4499 40.5921) (width 0.25) (layer "F.Cu") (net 23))
 (segment (start 61.29 39.9603) (end 64.725 36.5253) (width 0.25) (layer "F.Cu") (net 27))
 (segment (start 61.29 55.725) (end 61.29 39.9603) (width 0.25) (layer "F.Cu") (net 27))
 (segment (start 64.725 35.35) (end 64.725 36.5253) (width 0.25) (layer "F.Cu") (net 27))
 (segment (start 61.0042 35.9008) (end 80.5647 55.4613) (width 0.25) (layer "B.Cu") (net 19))
 (segment (start 61.8177 33.9853) (end 61.0042 34.7988) (width 0.25) (layer "B.Cu") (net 19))
 (segment (start 80.5647 55.4613) (end 80.5647 55.725) (width 0.25) (layer "B.Cu") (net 19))
 (segment (start 61.0042 34.7988) (end 61.0042 35.9008) (width 0.25) (layer "B.Cu") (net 19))
 (segment (start 81.61 55.725) (end 80.5647 55.725) (width 0.25) (layer "B.Cu") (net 19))
 (segment (start 62.185 32.81) (end 62.185 33.9853) (width 0.25) (layer "B.Cu") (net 19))
 (segment (start 62.185 33.9853) (end 61.8177 33.9853) (width 0.25) (layer "B.Cu") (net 19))
 (segment (start 83.1047 55.4314) (end 83.1047 55.725) (width 0.25) (layer "B.Cu") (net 18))
 (segment (start 84.15 55.725) (end 83.1047 55.725) (width 0.25) (layer "B.Cu") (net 18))
 (segment (start 80.7853 53.3267) (end 81 53.3267) (width 0.25) (layer "B.Cu") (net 18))
 (segment (start 81 53.3267) (end 83.1047 55.4314) (width 0.25) (layer "B.Cu") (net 18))
 (segment (start 63.3603 35.35) (end 63.3603 35.9017) (width 0.25) (layer "B.Cu") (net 18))
 (segment (start 63.3603 35.9017) (end 80.7853 53.3267) (width 0.25) (layer "B.Cu") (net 18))
 (segment (start 62.185 35.35) (end 63.3603 35.35) (width 0.25) (layer "B.Cu") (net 18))
 (segment (start 84.2132 51.4595) (end 88.1847 55.431) (width 0.25) (layer "B.Cu") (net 16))
 (segment (start 65.2027 31.6189) (end 65.9521 32.3683) (width 0.25) (layer "B.Cu") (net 16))
 (segment (start 65.9521 32.3683) (end 65.9521 37.7914) (width 0.25) (layer "B.Cu") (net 16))
 (segment (start 60.8203 32.81) (end 60.8203 32.4427) (width 0.25) (layer "B.Cu") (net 16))
 (segment (start 61.6441 31.6189) (end 65.2027 31.6189) (width 0.25) (layer "B.Cu") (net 16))
 (segment (start 60.8203 32.4427) (end 61.6441 31.6189) (width 0.25) (layer "B.Cu") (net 16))
 (segment (start 88.1847 55.431) (end 88.1847 55.725) (width 0.25) (layer "B.Cu") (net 16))
 (segment (start 79.6202 51.4595) (end 84.2132 51.4595) (width 0.25) (layer "B.Cu") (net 16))
 (segment (start 65.9521 37.7914) (end 79.6202 51.4595) (width 0.25) (layer "B.Cu") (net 16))
 (segment (start 89.23 55.725) (end 88.1847 55.725) (width 0.25) (layer "B.Cu") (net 16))
 (segment (start 59.645 32.81) (end 60.8203 32.81) (width 0.25) (layer "B.Cu") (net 16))
 (segment (start 86.2648 63.6711) (end 88.1847 65.591) (width 0.25) (layer "B.Cu") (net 13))
 (segment (start 57.105 33.9853) (end 57.4724 33.9853) (width 0.25) (layer "B.Cu") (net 13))
 (segment (start 57.105 32.81) (end 57.105 33.9853) (width 0.25) (layer "B.Cu") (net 13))
 (segment (start 88.1847 65.591) (end 88.1847 65.885) (width 0.25) (layer "B.Cu") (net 13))
 (segment (start 58.2803 35.7168) (end 77.8 55.2365) (width 0.25) (layer "B.Cu") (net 13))
 (segment (start 89.23 65.885) (end 88.1847 65.885) (width 0.25) (layer "B.Cu") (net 13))
 (segment (start 85.2142 63.6711) (end 86.2648 63.6711) (width 0.25) (layer "B.Cu") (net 13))
 (segment (start 77.8 56.2569) (end 85.2142 63.6711) (width 0.25) (layer "B.Cu") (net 13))
 (segment (start 57.4724 33.9853) (end 58.2803 34.7932) (width 0.25) (layer "B.Cu") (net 13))
 (segment (start 58.2803 34.7932) (end 58.2803 35.7168) (width 0.25) (layer "B.Cu") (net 13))
 (segment (start 77.8 55.2365) (end 77.8 56.2569) (width 0.25) (layer "B.Cu") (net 13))
 (segment (start 57.105 59.16) (end 62.7847 64.8397) (width 0.25) (layer "F.Cu") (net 3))
 (segment (start 62.7847 64.8397) (end 62.7847 65.885) (width 0.25) (layer "F.Cu") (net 3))
 (segment (start 63.83 65.885) (end 62.7847 65.885) (width 0.25) (layer "F.Cu") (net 3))
 (segment (start 57.105 35.35) (end 57.105 59.16) (width 0.25) (layer "F.Cu") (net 3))
 (segment (start 61.29 65.885) (end 60.2447 65.885) (width 0.25) (layer "B.Cu") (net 2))
 (segment (start 60.2447 42.205) (end 60.2447 65.885) (width 0.25) (layer "B.Cu") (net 2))
 (segment (start 54.565 35.35) (end 54.565 36.5253) (width 0.25) (layer "B.Cu") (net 2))
 (segment (start 54.565 36.5253) (end 60.2447 42.205) (width 0.25) (layer "B.Cu") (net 2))
 (segment (start 52.025 35.35) (end 52.025 60.2053) (width 0.25) (layer "B.Cu") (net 1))
 (segment (start 58.75 65.885) (end 57.7047 65.885) (width 0.25) (layer "B.Cu") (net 1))
 (segment (start 52.025 60.2053) (end 57.7047 65.885) (width 0.25) (layer "B.Cu") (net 1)))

